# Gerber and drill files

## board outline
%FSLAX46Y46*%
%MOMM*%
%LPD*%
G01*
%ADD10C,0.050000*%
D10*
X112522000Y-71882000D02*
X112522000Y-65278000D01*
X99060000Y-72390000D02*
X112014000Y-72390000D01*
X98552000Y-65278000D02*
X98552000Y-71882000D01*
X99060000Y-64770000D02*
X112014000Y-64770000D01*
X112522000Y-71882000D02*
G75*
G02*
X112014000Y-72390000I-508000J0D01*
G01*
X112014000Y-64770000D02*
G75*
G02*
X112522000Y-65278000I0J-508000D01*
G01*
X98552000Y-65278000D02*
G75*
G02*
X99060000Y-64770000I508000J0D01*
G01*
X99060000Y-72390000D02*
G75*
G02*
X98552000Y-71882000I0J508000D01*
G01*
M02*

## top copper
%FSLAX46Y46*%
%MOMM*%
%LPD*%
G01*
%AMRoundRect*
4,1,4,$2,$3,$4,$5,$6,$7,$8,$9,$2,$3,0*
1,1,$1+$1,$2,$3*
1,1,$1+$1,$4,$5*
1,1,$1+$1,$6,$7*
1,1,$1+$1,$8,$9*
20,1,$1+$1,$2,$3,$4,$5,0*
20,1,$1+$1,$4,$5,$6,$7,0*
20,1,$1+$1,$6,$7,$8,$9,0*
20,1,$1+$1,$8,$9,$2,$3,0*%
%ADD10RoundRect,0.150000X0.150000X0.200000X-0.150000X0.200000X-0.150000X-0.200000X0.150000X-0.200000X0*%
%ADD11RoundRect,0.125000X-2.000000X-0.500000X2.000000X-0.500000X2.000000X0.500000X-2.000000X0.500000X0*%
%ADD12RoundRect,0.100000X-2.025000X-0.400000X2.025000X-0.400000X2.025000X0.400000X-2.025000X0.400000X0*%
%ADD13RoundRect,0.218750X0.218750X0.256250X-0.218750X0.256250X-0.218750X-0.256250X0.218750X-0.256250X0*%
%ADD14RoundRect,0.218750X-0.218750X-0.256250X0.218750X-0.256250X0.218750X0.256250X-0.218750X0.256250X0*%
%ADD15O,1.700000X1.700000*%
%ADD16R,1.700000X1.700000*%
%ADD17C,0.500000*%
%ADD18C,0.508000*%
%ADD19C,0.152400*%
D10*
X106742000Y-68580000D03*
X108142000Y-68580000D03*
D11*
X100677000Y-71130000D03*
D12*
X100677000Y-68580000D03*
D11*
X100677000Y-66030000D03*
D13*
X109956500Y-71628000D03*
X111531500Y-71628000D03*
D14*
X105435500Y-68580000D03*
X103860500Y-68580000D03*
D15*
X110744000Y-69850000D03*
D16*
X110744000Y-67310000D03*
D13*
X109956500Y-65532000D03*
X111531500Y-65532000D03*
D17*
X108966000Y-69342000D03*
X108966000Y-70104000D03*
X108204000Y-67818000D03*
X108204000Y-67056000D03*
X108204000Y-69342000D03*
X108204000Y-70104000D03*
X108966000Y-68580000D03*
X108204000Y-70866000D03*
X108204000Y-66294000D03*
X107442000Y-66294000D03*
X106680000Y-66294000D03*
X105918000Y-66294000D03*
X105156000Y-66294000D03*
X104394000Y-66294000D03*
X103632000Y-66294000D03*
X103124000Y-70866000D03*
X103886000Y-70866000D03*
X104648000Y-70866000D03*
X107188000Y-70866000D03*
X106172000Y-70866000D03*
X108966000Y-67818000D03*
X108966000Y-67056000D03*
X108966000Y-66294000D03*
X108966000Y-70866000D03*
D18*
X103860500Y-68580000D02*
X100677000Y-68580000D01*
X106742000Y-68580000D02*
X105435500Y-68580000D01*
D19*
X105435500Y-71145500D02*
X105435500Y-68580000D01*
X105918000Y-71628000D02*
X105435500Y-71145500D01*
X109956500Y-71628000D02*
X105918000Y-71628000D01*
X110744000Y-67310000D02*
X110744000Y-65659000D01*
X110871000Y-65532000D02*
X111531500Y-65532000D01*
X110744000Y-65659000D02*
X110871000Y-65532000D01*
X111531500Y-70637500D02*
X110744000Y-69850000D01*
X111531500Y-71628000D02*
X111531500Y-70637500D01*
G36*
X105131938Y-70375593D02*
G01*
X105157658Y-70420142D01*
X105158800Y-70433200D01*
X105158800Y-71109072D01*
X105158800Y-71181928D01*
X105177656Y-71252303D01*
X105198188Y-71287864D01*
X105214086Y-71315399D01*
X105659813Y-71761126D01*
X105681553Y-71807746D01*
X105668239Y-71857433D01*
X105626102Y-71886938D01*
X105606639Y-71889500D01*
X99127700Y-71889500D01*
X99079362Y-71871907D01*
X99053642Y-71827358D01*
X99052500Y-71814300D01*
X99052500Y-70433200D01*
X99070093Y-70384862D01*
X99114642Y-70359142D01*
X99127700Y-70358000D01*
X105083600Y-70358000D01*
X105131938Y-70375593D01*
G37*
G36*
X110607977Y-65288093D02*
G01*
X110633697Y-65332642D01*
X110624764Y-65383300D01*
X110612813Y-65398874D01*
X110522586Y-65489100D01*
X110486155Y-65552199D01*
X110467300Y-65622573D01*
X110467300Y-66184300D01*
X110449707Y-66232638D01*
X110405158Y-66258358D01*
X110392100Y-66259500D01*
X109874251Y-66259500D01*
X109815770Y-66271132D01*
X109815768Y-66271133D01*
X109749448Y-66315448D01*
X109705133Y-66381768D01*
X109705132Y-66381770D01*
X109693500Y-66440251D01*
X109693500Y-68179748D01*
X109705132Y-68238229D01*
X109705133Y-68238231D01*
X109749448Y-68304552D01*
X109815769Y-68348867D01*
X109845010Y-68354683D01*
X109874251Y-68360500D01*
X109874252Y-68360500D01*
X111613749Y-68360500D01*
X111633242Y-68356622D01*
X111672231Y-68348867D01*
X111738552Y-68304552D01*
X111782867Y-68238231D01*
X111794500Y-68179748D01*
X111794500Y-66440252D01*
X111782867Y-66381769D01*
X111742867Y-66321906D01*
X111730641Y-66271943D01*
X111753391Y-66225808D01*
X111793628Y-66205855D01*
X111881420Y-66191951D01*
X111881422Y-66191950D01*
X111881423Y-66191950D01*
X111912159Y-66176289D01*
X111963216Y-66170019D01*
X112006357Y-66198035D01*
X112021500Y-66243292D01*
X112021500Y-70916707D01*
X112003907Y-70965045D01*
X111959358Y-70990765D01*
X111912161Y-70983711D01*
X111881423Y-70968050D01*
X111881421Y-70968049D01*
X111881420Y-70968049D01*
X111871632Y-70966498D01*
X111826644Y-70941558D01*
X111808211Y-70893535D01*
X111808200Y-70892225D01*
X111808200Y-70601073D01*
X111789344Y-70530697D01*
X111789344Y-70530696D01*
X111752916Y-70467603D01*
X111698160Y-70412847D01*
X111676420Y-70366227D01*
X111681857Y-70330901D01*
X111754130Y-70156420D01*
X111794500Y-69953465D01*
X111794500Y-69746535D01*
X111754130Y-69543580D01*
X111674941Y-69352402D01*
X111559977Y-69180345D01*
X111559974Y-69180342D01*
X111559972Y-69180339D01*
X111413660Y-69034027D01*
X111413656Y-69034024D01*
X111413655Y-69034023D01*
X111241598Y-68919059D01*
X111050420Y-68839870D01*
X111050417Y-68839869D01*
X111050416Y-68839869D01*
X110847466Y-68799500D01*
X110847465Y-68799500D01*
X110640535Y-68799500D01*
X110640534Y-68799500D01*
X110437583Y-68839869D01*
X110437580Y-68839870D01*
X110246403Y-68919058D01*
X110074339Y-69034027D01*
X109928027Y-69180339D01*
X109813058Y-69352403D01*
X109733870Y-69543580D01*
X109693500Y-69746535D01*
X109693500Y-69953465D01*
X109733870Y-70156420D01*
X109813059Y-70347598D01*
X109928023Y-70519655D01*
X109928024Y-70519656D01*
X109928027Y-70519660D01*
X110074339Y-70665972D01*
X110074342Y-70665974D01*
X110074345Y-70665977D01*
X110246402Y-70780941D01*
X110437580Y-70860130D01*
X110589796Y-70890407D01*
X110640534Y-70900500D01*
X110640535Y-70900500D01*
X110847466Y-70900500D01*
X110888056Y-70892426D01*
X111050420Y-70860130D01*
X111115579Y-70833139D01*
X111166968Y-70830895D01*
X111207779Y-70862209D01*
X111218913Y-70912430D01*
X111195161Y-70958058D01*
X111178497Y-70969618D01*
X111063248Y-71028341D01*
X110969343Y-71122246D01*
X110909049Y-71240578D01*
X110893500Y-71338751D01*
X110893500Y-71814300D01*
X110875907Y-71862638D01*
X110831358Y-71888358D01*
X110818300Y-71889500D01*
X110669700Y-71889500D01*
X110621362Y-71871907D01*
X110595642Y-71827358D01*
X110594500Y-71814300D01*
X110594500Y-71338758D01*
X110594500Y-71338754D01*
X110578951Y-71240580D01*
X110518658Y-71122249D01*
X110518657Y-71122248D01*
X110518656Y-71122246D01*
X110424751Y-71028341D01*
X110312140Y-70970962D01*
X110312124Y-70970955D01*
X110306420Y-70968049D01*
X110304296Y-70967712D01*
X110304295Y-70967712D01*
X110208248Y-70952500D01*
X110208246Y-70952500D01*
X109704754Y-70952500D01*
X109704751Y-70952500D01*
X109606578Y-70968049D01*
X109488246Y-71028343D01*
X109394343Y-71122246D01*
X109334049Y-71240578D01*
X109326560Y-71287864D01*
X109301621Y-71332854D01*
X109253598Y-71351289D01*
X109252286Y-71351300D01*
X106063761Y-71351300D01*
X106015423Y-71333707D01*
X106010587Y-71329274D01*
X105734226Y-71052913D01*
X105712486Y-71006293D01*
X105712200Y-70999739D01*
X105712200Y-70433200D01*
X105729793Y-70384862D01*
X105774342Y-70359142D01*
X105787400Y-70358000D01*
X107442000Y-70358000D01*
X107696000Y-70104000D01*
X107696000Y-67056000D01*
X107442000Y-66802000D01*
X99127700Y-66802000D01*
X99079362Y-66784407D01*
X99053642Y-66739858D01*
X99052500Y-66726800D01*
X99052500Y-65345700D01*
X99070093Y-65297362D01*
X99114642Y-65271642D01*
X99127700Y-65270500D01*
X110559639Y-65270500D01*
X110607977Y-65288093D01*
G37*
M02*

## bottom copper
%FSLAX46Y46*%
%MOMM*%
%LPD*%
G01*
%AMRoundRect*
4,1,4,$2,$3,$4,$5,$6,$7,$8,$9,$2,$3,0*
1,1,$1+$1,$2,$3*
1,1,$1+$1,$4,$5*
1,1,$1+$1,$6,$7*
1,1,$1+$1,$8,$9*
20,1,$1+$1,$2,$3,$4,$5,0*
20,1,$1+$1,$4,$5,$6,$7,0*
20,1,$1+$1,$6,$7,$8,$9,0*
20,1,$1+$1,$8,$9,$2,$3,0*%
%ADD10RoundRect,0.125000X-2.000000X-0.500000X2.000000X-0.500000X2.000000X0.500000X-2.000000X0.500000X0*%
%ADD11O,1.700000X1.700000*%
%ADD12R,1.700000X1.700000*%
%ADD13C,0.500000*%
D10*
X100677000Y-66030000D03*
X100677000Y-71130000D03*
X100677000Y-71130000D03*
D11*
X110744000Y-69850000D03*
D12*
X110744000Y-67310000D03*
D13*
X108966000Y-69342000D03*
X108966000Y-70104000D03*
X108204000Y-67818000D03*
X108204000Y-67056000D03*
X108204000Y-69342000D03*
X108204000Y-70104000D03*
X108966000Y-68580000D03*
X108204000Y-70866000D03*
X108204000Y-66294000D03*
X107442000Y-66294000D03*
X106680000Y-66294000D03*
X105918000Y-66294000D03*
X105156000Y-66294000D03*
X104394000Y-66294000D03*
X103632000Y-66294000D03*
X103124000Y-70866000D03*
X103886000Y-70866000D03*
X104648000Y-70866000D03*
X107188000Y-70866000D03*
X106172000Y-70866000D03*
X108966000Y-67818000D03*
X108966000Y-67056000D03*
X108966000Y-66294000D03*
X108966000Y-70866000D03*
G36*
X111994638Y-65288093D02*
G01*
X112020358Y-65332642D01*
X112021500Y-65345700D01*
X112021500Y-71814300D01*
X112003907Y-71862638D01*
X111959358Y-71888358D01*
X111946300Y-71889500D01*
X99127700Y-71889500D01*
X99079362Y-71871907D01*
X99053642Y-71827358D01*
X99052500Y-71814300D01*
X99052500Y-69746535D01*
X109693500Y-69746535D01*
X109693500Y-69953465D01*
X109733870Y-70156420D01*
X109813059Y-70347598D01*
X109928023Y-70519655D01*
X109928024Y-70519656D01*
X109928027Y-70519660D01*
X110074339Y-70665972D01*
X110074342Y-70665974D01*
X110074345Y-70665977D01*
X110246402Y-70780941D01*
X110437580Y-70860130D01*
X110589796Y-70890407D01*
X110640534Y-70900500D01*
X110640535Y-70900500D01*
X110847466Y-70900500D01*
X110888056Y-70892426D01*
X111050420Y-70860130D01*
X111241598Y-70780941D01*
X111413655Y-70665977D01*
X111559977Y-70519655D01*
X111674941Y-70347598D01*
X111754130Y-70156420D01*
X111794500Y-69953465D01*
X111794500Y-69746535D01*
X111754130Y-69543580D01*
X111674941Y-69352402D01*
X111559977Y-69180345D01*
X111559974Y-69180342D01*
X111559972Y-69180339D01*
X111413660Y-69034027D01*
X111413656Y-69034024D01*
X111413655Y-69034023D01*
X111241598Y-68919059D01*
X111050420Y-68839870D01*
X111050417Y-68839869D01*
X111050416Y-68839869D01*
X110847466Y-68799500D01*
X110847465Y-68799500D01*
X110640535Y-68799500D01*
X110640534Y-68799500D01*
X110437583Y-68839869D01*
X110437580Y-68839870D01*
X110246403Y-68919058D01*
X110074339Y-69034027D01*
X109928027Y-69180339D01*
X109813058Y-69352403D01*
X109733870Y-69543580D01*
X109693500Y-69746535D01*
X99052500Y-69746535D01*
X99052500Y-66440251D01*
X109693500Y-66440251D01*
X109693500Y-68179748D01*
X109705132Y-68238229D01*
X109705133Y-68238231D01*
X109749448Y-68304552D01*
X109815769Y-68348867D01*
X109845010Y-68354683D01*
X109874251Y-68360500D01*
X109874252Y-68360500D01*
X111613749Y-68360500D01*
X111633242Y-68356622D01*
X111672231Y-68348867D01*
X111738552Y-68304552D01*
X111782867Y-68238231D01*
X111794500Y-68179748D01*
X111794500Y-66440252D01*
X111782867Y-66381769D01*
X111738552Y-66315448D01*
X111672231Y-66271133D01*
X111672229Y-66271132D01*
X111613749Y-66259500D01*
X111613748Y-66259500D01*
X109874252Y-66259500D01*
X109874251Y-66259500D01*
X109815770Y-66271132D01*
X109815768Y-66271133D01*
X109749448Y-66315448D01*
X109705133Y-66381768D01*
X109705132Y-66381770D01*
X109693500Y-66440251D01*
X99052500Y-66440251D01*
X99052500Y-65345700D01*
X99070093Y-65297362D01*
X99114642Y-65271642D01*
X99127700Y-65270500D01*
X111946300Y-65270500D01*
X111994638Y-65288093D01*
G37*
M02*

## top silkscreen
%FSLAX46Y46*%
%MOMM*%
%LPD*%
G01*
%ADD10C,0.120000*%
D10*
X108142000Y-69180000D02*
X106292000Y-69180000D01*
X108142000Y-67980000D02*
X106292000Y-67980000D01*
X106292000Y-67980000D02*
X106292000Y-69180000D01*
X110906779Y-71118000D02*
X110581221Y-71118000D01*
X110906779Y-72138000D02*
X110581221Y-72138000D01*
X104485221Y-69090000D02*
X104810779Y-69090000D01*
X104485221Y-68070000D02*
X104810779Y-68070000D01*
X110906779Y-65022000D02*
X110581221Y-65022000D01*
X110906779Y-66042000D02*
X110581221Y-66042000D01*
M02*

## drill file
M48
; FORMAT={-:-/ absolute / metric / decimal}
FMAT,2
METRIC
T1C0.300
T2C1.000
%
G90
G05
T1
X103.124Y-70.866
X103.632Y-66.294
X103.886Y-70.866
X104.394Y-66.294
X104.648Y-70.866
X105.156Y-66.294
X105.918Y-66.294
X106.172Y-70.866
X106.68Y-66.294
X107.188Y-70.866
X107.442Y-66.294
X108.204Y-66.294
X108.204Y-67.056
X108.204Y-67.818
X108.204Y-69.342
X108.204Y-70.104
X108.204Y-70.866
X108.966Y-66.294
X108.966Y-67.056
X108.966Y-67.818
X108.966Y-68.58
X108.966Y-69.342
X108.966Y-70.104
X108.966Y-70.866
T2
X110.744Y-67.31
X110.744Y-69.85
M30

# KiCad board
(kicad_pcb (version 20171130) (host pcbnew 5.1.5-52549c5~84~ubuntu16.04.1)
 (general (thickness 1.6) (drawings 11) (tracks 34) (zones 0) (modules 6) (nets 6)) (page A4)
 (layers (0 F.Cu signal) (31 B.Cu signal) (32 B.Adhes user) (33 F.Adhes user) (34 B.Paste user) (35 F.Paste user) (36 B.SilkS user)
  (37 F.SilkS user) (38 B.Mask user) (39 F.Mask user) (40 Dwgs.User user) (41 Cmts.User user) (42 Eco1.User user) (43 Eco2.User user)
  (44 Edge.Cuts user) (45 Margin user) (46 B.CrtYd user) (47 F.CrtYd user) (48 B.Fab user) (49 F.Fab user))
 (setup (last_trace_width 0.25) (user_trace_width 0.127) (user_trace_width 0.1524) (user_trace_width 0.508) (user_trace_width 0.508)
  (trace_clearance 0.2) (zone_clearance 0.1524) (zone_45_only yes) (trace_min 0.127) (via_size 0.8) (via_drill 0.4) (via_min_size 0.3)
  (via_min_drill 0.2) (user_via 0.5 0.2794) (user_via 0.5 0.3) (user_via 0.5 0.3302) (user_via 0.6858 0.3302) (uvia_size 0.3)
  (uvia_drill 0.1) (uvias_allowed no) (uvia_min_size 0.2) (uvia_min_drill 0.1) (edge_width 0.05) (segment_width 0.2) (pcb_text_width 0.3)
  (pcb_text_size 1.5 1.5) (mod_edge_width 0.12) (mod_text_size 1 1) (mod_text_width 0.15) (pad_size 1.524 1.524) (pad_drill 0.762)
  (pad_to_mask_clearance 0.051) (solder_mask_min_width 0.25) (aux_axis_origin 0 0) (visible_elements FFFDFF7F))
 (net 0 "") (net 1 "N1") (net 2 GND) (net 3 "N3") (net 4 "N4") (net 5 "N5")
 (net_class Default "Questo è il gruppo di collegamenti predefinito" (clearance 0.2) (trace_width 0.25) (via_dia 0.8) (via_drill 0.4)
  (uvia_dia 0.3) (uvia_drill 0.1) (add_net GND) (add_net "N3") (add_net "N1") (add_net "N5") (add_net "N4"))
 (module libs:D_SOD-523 (layer F.Cu) (at 107.442 68.58)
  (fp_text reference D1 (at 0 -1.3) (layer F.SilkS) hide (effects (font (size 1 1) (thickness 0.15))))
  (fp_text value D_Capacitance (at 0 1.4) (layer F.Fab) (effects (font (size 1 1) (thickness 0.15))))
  (fp_line (start 0.7 0.6) (end -1.15 0.6) (layer F.SilkS) (width 0.12))
  (fp_line (start 0.7 -0.6) (end -1.15 -0.6) (layer F.SilkS) (width 0.12))
  (fp_line (start -1.15 -0.6) (end -1.15 0.6) (layer F.SilkS) (width 0.12))
  (pad 1 smd roundrect (at -0.7 0 180) (size 0.6 0.7) (layers F.Cu F.Paste F.Mask) (roundrect_rratio 0.25) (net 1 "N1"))
  (pad 2 smd roundrect (at 0.7 0 180) (size 0.6 0.7) (layers F.Cu F.Paste F.Mask) (roundrect_rratio 0.25) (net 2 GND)))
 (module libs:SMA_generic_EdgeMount (layer F.Cu) (at 98.552 68.58)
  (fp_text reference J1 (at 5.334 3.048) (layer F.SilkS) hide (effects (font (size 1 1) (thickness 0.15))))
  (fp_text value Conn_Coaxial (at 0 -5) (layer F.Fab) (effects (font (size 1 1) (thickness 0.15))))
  (pad 2 smd roundrect (at 2.125 -2.55) (size 4.25 1.25) (layers B.Cu B.Paste B.Mask) (roundrect_rratio 0.1) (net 2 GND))
  (pad 2 smd roundrect (at 2.125 2.55) (size 4.25 1.25) (layers F.Cu F.Paste F.Mask) (roundrect_rratio 0.1) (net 2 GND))
  (pad 2 smd roundrect (at 2.125 2.55) (size 4.25 1.25) (layers B.Cu B.Paste B.Mask) (roundrect_rratio 0.1) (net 2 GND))
  (pad 1 smd roundrect (at 2.125 0) (size 4.25 1) (layers F.Cu F.Paste F.Mask) (roundrect_rratio 0.1) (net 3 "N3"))
  (pad 2 smd roundrect (at 2.125 -2.55) (size 4.25 1.25) (layers F.Cu F.Paste F.Mask) (roundrect_rratio 0.1) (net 2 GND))
  (pad 2 smd roundrect (at 2.125 2.55) (size 4.25 1.25) (layers B.Cu B.Paste B.Mask) (roundrect_rratio 0.1) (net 2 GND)))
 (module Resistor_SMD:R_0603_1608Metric (layer F.Cu) (at 110.744 71.628 180)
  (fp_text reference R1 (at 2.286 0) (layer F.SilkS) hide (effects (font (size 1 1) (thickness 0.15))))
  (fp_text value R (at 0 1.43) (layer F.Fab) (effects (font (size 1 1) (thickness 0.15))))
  (fp_line (start -0.162779 0.51) (end 0.162779 0.51) (layer F.SilkS) (width 0.12))
  (fp_line (start -0.162779 -0.51) (end 0.162779 -0.51) (layer F.SilkS) (width 0.12))
  (pad 2 smd roundrect (at 0.7875 0 180) (size 0.875 0.95) (layers F.Cu F.Paste F.Mask) (roundrect_rratio 0.25) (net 1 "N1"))
  (pad 1 smd roundrect (at -0.7875 0 180) (size 0.875 0.95) (layers F.Cu F.Paste F.Mask) (roundrect_rratio 0.25) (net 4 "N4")))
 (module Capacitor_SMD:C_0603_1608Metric (layer F.Cu) (at 104.648 68.58)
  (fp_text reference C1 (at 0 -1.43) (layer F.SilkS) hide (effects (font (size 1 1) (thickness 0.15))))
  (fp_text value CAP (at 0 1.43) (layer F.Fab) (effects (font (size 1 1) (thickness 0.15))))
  (fp_line (start -0.162779 0.51) (end 0.162779 0.51) (layer F.SilkS) (width 0.12))
  (fp_line (start -0.162779 -0.51) (end 0.162779 -0.51) (layer F.SilkS) (width 0.12))
  (pad 2 smd roundrect (at 0.7875 0) (size 0.875 0.95) (layers F.Cu F.Paste F.Mask) (roundrect_rratio 0.25) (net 1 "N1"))
  (pad 1 smd roundrect (at -0.7875 0) (size 0.875 0.95) (layers F.Cu F.Paste F.Mask) (roundrect_rratio 0.25) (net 3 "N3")))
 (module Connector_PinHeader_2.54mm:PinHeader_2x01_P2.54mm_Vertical (layer B.Cu) (at 110.744 67.31 270)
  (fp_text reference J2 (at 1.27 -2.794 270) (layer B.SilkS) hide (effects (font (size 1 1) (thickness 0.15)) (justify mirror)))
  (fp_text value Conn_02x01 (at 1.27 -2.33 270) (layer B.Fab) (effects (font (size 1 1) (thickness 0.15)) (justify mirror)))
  (pad 2 thru_hole oval (at 2.54 0 270) (size 1.7 1.7) (drill 1) (layers *.Cu *.Mask) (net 4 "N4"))
  (pad 1 thru_hole rect (at 0 0 270) (size 1.7 1.7) (drill 1) (layers *.Cu *.Mask) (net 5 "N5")))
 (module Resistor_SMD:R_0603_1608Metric (layer F.Cu) (at 110.744 65.532 180)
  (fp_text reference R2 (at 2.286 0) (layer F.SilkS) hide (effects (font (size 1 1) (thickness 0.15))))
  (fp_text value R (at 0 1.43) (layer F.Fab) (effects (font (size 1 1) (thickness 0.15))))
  (fp_line (start -0.162779 0.51) (end 0.162779 0.51) (layer F.SilkS) (width 0.12))
  (fp_line (start -0.162779 -0.51) (end 0.162779 -0.51) (layer F.SilkS) (width 0.12))
  (pad 2 smd roundrect (at 0.7875 0 180) (size 0.875 0.95) (layers F.Cu F.Paste F.Mask) (roundrect_rratio 0.25) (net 2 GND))
  (pad 1 smd roundrect (at -0.7875 0 180) (size 0.875 0.95) (layers F.Cu F.Paste F.Mask) (roundrect_rratio 0.25) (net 5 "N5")))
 (gr_line (start 112.522 71.882) (end 112.522 65.278) (layer Edge.Cuts) (width 0.05))
 (gr_line (start 99.06 72.39) (end 112.014 72.39) (layer Edge.Cuts) (width 0.05))
 (gr_line (start 98.552 65.278) (end 98.552 71.882) (layer Edge.Cuts) (width 0.05))
 (gr_line (start 99.06 64.77) (end 112.014 64.77) (layer Edge.Cuts) (width 0.05))
 (gr_arc (start 112.014 71.882) (end 112.014 72.39) (angle -90) (layer Edge.Cuts) (width 0.05))
 (gr_arc (start 112.014 65.278) (end 112.522 65.278) (angle -90) (layer Edge.Cuts) (width 0.05))
 (gr_arc (start 99.06 65.278) (end 99.06 64.77) (angle -90) (layer Edge.Cuts) (width 0.05))
 (gr_arc (start 99.06 71.882) (end 98.552 71.882) (angle -90) (layer Edge.Cuts) (width 0.05))
 (segment (start 103.8605 68.58) (end 100.677 68.58) (width 0.508) (layer F.Cu) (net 3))
 (segment (start 106.742 68.58) (end 105.4355 68.58) (width 0.508) (layer F.Cu) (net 1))
 (segment (start 105.4355 71.1455) (end 105.4355 68.58) (width 0.1524) (layer F.Cu) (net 1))
 (segment (start 105.918 71.628) (end 105.4355 71.1455) (width 0.1524) (layer F.Cu) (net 1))
 (segment (start 109.9565 71.628) (end 105.918 71.628) (width 0.1524) (layer F.Cu) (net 1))
 (via (at 108.966 69.342) (size 0.5) (drill 0.3) (layers F.Cu B.Cu) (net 2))
 (via (at 108.966 70.104) (size 0.5) (drill 0.3) (layers F.Cu B.Cu) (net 2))
 (via (at 108.204 67.818) (size 0.5) (drill 0.3) (layers F.Cu B.Cu) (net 2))
 (via (at 108.204 67.056) (size 0.5) (drill 0.3) (layers F.Cu B.Cu) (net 2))
 (via (at 108.204 69.342) (size 0.5) (drill 0.3) (layers F.Cu B.Cu) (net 2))
 (via (at 108.204 70.104) (size 0.5) (drill 0.3) (layers F.Cu B.Cu) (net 2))
 (via (at 108.966 68.58) (size 0.5) (drill 0.3) (layers F.Cu B.Cu) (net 2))
 (via (at 108.204 70.866) (size 0.5) (drill 0.3) (layers F.Cu B.Cu) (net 2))
 (via (at 108.204 66.294) (size 0.5) (drill 0.3) (layers F.Cu B.Cu) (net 2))
 (via (at 107.442 66.294) (size 0.5) (drill 0.3) (layers F.Cu B.Cu) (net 2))
 (via (at 106.68 66.294) (size 0.5) (drill 0.3) (layers F.Cu B.Cu) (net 2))
 (via (at 105.918 66.294) (size 0.5) (drill 0.3) (layers F.Cu B.Cu) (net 2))
 (via (at 105.156 66.294) (size 0.5) (drill 0.3) (layers F.Cu B.Cu) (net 2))
 (via (at 104.394 66.294) (size 0.5) (drill 0.3) (layers F.Cu B.Cu) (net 2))
 (via (at 103.632 66.294) (size 0.5) (drill 0.3) (layers F.Cu B.Cu) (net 2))
 (via (at 103.124 70.866) (size 0.5) (drill 0.3) (layers F.Cu B.Cu) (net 2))
 (via (at 103.886 70.866) (size 0.5) (drill 0.3) (layers F.Cu B.Cu) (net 2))
 (via (at 104.648 70.866) (size 0.5) (drill 0.3) (layers F.Cu B.Cu) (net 2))
 (via (at 107.188 70.866) (size 0.5) (drill 0.3) (layers F.Cu B.Cu) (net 2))
 (via (at 106.172 70.866) (size 0.5) (drill 0.3) (layers F.Cu B.Cu) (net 2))
 (via (at 108.966 67.818) (size 0.5) (drill 0.3) (layers F.Cu B.Cu) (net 2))
 (via (at 108.966 67.056) (size 0.5) (drill 0.3) (layers F.Cu B.Cu) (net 2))
 (via (at 108.966 66.294) (size 0.5) (drill 0.3) (layers F.Cu B.Cu) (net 2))
 (via (at 108.966 70.866) (size 0.5) (drill 0.3) (layers F.Cu B.Cu) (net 2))
 (segment (start 110.744 67.31) (end 110.744 65.659) (width 0.1524) (layer F.Cu) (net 5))
 (segment (start 110.871 65.532) (end 111.5315 65.532) (width 0.1524) (layer F.Cu) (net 5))
 (segment (start 110.744 65.659) (end 110.871 65.532) (width 0.1524) (layer F.Cu) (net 5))
 (segment (start 111.5315 70.6375) (end 110.744 69.85) (width 0.1524) (layer F.Cu) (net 4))
 (segment (start 111.5315 71.628) (end 111.5315 70.6375) (width 0.1524) (layer F.Cu) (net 4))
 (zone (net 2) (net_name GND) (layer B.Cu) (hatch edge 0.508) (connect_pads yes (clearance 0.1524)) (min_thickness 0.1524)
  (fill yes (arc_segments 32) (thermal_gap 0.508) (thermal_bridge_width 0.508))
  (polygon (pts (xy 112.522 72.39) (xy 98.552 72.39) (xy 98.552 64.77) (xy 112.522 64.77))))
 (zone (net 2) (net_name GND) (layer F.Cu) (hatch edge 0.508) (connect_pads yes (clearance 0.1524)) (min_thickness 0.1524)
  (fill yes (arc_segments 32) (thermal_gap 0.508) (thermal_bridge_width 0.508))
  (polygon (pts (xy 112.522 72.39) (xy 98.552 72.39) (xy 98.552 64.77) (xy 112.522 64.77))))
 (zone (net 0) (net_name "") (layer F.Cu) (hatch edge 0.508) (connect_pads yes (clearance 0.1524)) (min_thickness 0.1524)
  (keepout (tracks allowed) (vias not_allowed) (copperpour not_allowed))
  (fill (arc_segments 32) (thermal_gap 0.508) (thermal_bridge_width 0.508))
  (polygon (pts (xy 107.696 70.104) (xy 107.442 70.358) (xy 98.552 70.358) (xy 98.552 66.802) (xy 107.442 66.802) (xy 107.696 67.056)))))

